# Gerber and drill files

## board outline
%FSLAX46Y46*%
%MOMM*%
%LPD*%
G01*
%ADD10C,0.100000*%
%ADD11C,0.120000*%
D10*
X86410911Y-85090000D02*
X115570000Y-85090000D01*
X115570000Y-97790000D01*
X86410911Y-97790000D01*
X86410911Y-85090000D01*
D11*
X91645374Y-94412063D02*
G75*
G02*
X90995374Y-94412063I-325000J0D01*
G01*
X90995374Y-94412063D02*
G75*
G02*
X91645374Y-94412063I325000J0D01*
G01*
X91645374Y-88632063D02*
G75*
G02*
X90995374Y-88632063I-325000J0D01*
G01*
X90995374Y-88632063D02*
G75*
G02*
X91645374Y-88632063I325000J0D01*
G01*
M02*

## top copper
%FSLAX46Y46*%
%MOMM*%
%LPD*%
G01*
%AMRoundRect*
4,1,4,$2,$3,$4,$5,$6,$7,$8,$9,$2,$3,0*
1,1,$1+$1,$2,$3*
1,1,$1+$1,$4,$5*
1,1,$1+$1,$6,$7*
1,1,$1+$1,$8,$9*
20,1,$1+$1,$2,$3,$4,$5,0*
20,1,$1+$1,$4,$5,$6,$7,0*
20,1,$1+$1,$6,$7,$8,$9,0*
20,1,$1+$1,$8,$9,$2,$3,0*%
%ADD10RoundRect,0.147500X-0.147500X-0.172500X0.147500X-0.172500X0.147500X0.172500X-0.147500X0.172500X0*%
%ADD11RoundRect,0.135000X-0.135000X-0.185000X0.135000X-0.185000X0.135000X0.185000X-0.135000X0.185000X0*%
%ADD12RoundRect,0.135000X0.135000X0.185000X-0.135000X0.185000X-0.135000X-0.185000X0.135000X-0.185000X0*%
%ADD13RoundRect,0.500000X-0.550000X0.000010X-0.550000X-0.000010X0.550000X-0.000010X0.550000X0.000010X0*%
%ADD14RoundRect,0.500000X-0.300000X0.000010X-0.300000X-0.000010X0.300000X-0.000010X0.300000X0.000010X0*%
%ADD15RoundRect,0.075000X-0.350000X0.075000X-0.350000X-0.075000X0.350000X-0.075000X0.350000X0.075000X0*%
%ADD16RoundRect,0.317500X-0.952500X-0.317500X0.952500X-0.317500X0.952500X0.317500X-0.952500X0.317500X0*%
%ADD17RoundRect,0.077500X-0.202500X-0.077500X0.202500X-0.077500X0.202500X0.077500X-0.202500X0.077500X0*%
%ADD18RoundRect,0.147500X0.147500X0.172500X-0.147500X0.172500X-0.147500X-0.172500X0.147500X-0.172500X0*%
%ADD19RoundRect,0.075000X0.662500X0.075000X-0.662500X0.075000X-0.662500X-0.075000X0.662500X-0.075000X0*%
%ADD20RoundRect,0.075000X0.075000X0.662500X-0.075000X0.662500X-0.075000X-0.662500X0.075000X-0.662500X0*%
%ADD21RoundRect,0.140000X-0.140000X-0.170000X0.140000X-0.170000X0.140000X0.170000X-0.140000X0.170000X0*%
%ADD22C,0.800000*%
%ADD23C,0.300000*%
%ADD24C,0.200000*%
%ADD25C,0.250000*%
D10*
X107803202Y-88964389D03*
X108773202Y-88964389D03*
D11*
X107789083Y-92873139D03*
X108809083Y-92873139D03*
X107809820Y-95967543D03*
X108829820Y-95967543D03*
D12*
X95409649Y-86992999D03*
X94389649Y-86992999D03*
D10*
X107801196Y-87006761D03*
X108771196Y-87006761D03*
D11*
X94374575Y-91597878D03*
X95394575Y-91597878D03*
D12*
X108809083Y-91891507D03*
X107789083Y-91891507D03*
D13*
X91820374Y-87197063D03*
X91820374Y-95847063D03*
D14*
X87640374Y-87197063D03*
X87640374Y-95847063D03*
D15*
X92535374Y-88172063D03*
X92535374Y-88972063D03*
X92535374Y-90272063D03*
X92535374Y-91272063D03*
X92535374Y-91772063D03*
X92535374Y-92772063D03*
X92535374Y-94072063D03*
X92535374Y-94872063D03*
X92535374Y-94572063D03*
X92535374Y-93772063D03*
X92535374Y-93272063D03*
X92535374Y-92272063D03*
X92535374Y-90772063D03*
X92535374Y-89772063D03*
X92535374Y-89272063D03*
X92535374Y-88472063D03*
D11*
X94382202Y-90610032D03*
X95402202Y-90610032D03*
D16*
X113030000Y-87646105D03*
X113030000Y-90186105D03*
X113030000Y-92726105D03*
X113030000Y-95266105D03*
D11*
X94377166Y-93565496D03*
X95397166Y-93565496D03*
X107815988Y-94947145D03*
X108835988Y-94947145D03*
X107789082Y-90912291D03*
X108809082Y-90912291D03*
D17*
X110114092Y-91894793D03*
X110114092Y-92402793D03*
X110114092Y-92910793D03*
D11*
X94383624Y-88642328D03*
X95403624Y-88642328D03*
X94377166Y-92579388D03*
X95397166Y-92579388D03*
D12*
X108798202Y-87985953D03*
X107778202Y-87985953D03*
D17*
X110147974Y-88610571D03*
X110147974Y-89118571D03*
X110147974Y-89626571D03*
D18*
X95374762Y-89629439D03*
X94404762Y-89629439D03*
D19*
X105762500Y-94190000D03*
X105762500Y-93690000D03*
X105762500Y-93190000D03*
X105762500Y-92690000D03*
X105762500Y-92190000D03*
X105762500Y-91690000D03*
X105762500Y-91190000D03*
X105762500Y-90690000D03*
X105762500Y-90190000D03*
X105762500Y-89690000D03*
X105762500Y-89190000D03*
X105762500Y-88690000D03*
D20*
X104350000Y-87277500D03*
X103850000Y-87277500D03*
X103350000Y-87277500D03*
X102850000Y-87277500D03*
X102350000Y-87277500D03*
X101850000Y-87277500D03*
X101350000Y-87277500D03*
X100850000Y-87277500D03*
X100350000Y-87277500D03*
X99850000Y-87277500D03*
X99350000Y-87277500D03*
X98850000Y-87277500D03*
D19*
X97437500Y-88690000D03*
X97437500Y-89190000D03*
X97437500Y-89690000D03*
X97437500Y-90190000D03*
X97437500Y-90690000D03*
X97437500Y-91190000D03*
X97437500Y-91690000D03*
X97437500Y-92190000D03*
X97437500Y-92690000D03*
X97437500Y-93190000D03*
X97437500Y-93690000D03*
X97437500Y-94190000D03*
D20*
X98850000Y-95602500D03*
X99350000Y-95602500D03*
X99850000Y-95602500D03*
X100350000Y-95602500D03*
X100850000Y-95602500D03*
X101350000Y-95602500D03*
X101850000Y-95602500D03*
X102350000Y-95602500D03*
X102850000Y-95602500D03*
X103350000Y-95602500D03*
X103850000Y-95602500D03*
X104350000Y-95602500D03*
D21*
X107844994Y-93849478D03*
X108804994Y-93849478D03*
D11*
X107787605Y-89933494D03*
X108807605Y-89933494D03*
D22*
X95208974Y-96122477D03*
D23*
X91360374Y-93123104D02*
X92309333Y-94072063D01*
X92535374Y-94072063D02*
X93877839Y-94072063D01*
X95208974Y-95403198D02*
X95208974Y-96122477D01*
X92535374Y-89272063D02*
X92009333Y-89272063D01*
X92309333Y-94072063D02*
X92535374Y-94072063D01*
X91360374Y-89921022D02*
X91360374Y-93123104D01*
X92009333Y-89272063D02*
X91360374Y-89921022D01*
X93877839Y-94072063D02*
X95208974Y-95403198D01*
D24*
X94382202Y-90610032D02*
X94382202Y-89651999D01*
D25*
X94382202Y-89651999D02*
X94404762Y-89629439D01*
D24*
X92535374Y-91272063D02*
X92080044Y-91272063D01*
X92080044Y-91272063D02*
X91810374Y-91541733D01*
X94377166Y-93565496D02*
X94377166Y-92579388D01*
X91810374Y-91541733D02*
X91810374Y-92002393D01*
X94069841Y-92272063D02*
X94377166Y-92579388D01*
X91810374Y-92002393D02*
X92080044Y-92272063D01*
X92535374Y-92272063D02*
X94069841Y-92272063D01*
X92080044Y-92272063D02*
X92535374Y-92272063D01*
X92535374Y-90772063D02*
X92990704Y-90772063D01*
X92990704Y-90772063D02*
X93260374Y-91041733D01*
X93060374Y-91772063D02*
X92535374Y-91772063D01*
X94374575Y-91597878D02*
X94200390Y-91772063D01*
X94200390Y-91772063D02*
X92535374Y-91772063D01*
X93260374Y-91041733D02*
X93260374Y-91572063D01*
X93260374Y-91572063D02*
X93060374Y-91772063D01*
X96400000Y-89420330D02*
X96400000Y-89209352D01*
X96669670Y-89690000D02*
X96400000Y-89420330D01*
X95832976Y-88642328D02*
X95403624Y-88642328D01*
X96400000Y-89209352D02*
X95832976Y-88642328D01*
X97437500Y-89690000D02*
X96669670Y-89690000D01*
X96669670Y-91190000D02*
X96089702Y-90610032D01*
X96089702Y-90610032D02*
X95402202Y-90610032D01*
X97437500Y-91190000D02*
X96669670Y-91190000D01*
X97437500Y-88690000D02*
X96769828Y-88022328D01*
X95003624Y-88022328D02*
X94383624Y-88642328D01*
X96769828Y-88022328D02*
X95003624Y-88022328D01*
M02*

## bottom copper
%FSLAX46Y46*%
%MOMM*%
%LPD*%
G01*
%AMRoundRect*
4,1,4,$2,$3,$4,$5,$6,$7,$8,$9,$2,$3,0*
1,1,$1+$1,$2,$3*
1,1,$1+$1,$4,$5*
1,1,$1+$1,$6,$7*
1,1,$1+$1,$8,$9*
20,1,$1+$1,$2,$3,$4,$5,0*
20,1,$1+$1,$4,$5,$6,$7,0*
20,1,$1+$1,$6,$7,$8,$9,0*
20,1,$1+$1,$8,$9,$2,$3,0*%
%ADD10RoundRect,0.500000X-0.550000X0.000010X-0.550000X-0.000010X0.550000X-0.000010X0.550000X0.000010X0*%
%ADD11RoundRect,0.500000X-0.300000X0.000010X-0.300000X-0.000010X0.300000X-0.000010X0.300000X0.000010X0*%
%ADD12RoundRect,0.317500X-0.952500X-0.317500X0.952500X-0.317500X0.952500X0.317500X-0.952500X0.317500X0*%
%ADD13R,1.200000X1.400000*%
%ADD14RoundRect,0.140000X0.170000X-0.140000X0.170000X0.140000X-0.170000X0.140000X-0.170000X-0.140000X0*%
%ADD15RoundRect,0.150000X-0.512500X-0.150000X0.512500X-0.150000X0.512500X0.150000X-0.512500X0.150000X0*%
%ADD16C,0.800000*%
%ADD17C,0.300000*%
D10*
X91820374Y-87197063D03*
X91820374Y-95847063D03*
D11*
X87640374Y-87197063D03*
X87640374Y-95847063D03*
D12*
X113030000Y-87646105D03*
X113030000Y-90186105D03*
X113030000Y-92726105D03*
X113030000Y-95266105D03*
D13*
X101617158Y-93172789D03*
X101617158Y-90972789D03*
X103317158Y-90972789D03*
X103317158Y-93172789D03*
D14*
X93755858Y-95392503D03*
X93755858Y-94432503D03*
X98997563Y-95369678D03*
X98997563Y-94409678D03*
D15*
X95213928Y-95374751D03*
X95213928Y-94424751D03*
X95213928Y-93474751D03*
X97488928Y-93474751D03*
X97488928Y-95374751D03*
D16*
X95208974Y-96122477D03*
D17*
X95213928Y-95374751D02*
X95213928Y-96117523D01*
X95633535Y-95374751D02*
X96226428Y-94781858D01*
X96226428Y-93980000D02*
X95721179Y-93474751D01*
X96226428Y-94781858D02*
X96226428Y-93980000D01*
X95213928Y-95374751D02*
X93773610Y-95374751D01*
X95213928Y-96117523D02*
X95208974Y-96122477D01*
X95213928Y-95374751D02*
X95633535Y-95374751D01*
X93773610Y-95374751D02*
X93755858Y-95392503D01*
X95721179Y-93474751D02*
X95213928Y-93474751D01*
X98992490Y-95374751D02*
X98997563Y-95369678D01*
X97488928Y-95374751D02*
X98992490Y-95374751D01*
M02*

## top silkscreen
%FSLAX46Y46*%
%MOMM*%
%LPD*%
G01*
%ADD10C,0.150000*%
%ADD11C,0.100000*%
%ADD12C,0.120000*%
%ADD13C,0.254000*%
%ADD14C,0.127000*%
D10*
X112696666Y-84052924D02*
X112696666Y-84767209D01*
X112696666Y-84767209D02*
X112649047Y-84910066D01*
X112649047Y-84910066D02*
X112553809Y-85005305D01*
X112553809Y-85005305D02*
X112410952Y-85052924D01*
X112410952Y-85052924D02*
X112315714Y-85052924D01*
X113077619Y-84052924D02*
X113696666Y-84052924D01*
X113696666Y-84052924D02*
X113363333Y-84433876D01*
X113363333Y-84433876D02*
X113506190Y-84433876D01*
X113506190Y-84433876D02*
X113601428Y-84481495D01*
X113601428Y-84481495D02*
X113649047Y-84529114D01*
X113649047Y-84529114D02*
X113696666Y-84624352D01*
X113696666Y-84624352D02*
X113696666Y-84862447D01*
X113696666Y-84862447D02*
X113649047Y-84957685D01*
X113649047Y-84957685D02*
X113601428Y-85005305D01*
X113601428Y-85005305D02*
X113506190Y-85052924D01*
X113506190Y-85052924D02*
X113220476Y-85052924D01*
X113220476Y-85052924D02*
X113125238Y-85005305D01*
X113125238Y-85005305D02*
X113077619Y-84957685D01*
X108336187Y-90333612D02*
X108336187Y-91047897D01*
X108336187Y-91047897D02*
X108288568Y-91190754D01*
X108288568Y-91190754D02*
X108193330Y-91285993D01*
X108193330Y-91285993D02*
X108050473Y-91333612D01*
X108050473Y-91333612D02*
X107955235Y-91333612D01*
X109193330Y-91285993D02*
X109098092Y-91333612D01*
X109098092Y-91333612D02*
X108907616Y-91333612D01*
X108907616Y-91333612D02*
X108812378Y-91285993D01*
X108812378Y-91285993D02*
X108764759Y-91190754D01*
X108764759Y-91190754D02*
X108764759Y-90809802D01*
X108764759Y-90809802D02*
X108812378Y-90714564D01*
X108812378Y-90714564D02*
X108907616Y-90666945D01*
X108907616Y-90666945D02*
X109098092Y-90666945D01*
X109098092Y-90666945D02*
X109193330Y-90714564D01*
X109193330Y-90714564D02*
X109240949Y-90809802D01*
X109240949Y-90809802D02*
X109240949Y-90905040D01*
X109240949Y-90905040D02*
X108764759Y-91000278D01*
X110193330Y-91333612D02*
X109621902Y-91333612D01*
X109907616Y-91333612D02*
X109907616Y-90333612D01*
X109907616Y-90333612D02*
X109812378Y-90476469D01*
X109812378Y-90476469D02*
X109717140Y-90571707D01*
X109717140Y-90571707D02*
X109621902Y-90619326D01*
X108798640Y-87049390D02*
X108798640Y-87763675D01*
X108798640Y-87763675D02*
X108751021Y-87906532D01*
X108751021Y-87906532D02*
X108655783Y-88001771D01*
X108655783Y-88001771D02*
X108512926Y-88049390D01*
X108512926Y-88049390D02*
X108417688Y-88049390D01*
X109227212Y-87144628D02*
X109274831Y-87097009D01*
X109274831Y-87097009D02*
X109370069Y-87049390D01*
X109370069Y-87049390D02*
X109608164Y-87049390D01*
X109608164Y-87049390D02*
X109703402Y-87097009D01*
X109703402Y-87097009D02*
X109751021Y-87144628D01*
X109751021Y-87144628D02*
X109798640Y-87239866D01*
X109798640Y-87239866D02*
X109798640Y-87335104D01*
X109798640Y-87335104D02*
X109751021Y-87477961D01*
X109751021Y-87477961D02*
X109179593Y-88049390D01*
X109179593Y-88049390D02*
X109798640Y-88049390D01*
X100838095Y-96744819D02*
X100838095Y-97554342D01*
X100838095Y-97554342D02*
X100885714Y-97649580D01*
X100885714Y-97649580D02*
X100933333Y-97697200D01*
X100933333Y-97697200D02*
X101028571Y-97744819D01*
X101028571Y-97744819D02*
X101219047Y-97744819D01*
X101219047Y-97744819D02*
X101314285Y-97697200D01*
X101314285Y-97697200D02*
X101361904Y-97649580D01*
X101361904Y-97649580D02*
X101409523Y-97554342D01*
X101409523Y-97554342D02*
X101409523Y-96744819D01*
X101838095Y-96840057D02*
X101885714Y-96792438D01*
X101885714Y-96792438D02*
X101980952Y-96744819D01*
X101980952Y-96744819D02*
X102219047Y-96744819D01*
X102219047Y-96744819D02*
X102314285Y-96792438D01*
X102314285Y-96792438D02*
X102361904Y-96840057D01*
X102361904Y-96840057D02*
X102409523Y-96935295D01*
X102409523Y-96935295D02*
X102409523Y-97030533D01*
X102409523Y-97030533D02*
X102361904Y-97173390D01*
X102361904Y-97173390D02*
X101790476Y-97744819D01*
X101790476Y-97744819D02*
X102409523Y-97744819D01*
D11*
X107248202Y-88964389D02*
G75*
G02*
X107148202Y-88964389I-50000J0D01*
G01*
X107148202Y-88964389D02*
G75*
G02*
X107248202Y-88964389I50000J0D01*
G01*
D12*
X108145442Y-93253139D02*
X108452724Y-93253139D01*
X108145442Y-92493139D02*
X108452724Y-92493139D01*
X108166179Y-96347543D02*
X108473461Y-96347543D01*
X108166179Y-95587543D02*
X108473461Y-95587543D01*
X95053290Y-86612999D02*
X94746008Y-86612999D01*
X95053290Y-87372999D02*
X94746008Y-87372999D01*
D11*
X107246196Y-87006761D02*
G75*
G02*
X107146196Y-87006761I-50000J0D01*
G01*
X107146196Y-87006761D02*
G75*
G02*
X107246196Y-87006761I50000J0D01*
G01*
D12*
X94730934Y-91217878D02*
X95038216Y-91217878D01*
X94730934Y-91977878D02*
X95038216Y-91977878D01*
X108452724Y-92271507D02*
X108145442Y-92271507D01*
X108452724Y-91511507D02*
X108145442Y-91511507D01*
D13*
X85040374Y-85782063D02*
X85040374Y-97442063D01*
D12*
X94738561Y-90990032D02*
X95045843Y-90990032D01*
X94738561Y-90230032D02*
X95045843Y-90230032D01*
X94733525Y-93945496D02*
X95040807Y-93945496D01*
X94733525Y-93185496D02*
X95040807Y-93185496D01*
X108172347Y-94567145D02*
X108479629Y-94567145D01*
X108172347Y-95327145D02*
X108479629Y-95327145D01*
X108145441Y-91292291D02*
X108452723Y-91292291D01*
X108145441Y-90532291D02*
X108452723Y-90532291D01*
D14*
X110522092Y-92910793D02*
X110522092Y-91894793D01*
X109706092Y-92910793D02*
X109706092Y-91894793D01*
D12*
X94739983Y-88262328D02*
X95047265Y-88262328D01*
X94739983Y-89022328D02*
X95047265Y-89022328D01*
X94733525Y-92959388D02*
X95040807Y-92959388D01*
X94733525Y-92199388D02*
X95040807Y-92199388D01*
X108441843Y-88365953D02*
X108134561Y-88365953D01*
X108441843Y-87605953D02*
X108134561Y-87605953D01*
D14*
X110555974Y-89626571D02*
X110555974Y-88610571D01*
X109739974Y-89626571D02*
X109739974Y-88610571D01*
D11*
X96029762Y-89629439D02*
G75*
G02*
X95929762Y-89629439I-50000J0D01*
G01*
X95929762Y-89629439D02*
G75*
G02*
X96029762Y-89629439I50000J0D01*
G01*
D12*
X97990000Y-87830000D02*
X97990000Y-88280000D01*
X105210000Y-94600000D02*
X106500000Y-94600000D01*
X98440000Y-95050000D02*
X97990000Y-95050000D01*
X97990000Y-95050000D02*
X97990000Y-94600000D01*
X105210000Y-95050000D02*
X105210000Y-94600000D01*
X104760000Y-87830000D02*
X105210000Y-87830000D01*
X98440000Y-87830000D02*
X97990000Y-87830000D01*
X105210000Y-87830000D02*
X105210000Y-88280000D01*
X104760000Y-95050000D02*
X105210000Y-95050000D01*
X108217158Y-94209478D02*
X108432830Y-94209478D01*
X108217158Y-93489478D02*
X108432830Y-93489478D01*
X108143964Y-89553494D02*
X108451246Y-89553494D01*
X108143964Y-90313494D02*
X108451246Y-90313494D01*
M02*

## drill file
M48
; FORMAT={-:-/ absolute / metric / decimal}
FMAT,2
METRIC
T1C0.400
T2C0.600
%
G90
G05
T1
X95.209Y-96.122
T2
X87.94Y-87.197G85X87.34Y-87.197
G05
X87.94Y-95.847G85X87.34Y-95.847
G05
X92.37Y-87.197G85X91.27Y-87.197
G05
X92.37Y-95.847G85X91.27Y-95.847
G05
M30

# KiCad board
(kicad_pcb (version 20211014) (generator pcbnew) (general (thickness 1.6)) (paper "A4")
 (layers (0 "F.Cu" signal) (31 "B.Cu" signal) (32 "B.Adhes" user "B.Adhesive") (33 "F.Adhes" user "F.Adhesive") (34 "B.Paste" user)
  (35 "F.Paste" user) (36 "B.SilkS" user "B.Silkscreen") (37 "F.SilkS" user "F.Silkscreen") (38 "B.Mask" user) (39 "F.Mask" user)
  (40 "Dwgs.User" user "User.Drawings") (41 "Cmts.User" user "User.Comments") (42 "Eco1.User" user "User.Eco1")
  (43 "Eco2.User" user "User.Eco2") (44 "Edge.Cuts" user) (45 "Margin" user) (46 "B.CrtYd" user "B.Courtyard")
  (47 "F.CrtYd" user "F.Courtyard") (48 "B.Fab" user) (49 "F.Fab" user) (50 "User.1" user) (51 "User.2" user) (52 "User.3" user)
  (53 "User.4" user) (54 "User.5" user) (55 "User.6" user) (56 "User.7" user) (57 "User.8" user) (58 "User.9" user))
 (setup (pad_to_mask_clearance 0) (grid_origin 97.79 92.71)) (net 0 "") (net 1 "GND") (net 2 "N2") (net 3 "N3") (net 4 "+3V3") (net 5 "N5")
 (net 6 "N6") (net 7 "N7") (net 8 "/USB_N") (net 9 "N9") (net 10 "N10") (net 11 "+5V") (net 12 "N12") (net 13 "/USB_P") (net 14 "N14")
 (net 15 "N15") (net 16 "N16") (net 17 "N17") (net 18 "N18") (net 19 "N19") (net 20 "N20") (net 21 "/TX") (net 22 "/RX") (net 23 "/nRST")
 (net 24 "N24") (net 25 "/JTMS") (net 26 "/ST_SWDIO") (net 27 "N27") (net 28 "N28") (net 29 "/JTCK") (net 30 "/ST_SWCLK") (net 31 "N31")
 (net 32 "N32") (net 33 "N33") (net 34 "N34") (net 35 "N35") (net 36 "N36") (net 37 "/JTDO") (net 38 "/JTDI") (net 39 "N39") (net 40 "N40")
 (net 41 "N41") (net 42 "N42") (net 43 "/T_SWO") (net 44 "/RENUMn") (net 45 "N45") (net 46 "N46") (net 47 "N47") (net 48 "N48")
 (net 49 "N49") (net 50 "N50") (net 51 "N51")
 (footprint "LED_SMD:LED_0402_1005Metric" (layer "F.Cu") (at 108.288202 88.964389)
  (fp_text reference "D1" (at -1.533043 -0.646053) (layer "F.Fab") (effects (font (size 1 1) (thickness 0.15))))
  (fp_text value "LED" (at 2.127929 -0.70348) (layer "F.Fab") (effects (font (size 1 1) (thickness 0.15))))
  (fp_circle (center -1.09 0) (end -1.04 0) (layer "F.SilkS") (width 0.1) (fill none))
  (pad "1" smd roundrect (at -0.485 0) (size 0.59 0.64) (layers "F.Cu" "F.Paste" "F.Mask") (roundrect_rratio 0.25) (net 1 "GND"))
  (pad "2" smd roundrect (at 0.485 0) (size 0.59 0.64) (layers "F.Cu" "F.Paste" "F.Mask") (roundrect_rratio 0.25) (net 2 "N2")))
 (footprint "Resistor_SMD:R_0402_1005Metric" (layer "F.Cu") (at 108.299083 92.873139)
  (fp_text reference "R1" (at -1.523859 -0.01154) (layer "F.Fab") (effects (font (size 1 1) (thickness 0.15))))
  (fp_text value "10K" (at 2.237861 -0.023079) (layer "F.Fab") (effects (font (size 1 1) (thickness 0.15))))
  (fp_line (start -0.153641 0.38) (end 0.153641 0.38) (layer "F.SilkS") (width 0.12))
  (fp_line (start -0.153641 -0.38) (end 0.153641 -0.38) (layer "F.SilkS") (width 0.12))
  (pad "1" smd roundrect (at -0.51 0) (size 0.54 0.64) (layers "F.Cu" "F.Paste" "F.Mask") (roundrect_rratio 0.25) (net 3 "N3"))
  (pad "2" smd roundrect (at 0.51 0) (size 0.54 0.64) (layers "F.Cu" "F.Paste" "F.Mask") (roundrect_rratio 0.25) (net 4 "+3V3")))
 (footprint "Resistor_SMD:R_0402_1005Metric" (layer "F.Cu") (at 108.31982 95.967543)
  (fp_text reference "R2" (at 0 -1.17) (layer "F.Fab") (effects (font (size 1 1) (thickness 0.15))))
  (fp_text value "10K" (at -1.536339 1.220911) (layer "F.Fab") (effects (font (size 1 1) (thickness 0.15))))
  (fp_line (start -0.153641 0.38) (end 0.153641 0.38) (layer "F.SilkS") (width 0.12))
  (fp_line (start -0.153641 -0.38) (end 0.153641 -0.38) (layer "F.SilkS") (width 0.12))
  (pad "1" smd roundrect (at -0.51 0) (size 0.54 0.64) (layers "F.Cu" "F.Paste" "F.Mask") (roundrect_rratio 0.25) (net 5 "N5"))
  (pad "2" smd roundrect (at 0.51 0) (size 0.54 0.64) (layers "F.Cu" "F.Paste" "F.Mask") (roundrect_rratio 0.25) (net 1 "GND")))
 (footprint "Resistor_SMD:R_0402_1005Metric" (layer "F.Cu") (at 94.899649 86.992999 180)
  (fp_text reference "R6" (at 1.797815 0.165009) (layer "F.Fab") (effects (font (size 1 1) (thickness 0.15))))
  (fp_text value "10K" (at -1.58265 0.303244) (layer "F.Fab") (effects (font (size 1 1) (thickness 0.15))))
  (fp_line (start -0.153641 0.38) (end 0.153641 0.38) (layer "F.SilkS") (width 0.12))
  (fp_line (start -0.153641 -0.38) (end 0.153641 -0.38) (layer "F.SilkS") (width 0.12))
  (pad "1" smd roundrect (at -0.51 0 180) (size 0.54 0.64) (layers "F.Cu" "F.Paste" "F.Mask") (roundrect_rratio 0.25) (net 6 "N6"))
  (pad "2" smd roundrect (at 0.51 0 180) (size 0.54 0.64) (layers "F.Cu" "F.Paste" "F.Mask") (roundrect_rratio 0.25) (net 1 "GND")))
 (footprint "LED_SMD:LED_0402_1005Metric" (layer "F.Cu") (at 108.286196 87.006761)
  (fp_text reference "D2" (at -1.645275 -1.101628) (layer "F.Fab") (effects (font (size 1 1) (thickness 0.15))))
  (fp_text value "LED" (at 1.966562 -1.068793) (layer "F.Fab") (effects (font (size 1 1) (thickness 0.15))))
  (fp_circle (center -1.09 0) (end -1.04 0) (layer "F.SilkS") (width 0.1) (fill none))
  (pad "1" smd roundrect (at -0.485 0) (size 0.59 0.64) (layers "F.Cu" "F.Paste" "F.Mask") (roundrect_rratio 0.25) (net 1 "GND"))
  (pad "2" smd roundrect (at 0.485 0) (size 0.59 0.64) (layers "F.Cu" "F.Paste" "F.Mask") (roundrect_rratio 0.25) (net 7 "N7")))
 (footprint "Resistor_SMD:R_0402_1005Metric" (layer "F.Cu") (at 94.884575 91.597878)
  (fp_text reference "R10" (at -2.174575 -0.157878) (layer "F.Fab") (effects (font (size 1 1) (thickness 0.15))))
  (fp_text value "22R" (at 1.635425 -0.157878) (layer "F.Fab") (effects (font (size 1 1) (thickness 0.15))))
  (fp_line (start -0.153641 -0.38) (end 0.153641 -0.38) (layer "F.SilkS") (width 0.12))
  (fp_line (start -0.153641 0.38) (end 0.153641 0.38) (layer "F.SilkS") (width 0.12))
  (pad "1" smd roundrect (at -0.51 0) (size 0.54 0.64) (layers "F.Cu" "F.Paste" "F.Mask") (roundrect_rratio 0.25) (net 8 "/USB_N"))
  (pad "2" smd roundrect (at 0.51 0) (size 0.54 0.64) (layers "F.Cu" "F.Paste" "F.Mask") (roundrect_rratio 0.25) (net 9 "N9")))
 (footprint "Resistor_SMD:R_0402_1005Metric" (layer "F.Cu") (at 108.299083 91.891507 180)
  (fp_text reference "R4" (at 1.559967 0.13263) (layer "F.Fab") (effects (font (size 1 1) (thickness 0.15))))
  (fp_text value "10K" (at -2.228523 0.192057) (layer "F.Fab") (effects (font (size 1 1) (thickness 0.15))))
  (fp_line (start -0.153641 -0.38) (end 0.153641 -0.38) (layer "F.SilkS") (width 0.12))
  (fp_line (start -0.153641 0.38) (end 0.153641 0.38) (layer "F.SilkS") (width 0.12))
  (pad "1" smd roundrect (at -0.51 0 180) (size 0.54 0.64) (layers "F.Cu" "F.Paste" "F.Mask") (roundrect_rratio 0.25) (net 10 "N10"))
  (pad "2" smd roundrect (at 0.51 0 180) (size 0.54 0.64) (layers "F.Cu" "F.Paste" "F.Mask") (roundrect_rratio 0.25) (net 4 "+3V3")))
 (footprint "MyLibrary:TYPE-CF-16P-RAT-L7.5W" (layer "F.Cu") (at 92.535374 88.322063 -90)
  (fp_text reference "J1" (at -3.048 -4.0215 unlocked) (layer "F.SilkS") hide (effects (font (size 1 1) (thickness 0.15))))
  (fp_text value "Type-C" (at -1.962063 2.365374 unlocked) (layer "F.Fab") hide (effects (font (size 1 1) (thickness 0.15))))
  (fp_line (start -2.54 7.495) (end 9.12 7.495) (layer "F.SilkS") (width 0.254))
  (fp_circle (center 6.09 1.215) (end 6.415 1.215) (layer "Edge.Cuts") (width 0.12) (fill none))
  (fp_circle (center 0.31 1.215) (end 0.635 1.215) (layer "Edge.Cuts") (width 0.12) (fill none))
  (pad "1" thru_hole roundrect (at -1.125 0.715 270) (size 1 2.1) (drill oval 0.6 1.7) (layers *.Cu *.Mask) (roundrect_rratio 0.5)
   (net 1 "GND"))
  (pad "2" thru_hole roundrect (at 7.525 0.715 270) (size 1 2.1) (drill oval 0.6 1.7) (layers *.Cu *.Mask) (roundrect_rratio 0.5)
   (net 1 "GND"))
  (pad "3" thru_hole roundrect (at -1.125 4.895 270) (size 1 1.6) (drill oval 0.6 1.2) (layers *.Cu *.Mask) (roundrect_rratio 0.5)
   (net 1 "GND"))
  (pad "4" thru_hole roundrect (at 7.525 4.895 270) (size 1 1.6) (drill oval 0.6 1.2) (layers *.Cu *.Mask) (roundrect_rratio 0.5)
   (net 1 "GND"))
  (pad "A1" smd roundrect (at -0.15 0 270) (size 0.3 0.85) (layers "F.Cu" "F.Paste" "F.Mask") (roundrect_rratio 0.25) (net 1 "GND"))
  (pad "A4" smd roundrect (at 0.65 0 270) (size 0.3 0.85) (layers "F.Cu" "F.Paste" "F.Mask") (roundrect_rratio 0.25) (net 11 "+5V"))
  (pad "A5" smd roundrect (at 1.95 0 270) (size 0.3 0.85) (layers "F.Cu" "F.Paste" "F.Mask") (roundrect_rratio 0.25) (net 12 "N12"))
  (pad "A6" smd roundrect (at 2.95 0 270) (size 0.3 0.85) (layers "F.Cu" "F.Paste" "F.Mask") (roundrect_rratio 0.25) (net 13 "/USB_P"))
  (pad "A7" smd roundrect (at 3.45 0 270) (size 0.3 0.85) (layers "F.Cu" "F.Paste" "F.Mask") (roundrect_rratio 0.25) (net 8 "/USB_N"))
  (pad "A8" smd roundrect (at 4.45 0 270) (size 0.3 0.85) (layers "F.Cu" "F.Paste" "F.Mask") (roundrect_rratio 0.25) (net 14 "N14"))
  (pad "A9" smd roundrect (at 5.75 0 270) (size 0.3 0.85) (layers "F.Cu" "F.Paste" "F.Mask") (roundrect_rratio 0.25) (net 11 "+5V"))
  (pad "A12" smd roundrect (at 6.55 0 270) (size 0.3 0.85) (layers "F.Cu" "F.Paste" "F.Mask") (roundrect_rratio 0.25) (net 1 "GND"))
  (pad "B1" smd roundrect (at 6.25 0 270) (size 0.3 0.85) (layers "F.Cu" "F.Paste" "F.Mask") (roundrect_rratio 0.25) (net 1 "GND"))
  (pad "B4" smd roundrect (at 5.45 0 270) (size 0.3 0.85) (layers "F.Cu" "F.Paste" "F.Mask") (roundrect_rratio 0.25) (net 11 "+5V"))
  (pad "B5" smd roundrect (at 4.95 0 270) (size 0.3 0.85) (layers "F.Cu" "F.Paste" "F.Mask") (roundrect_rratio 0.25) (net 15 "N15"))
  (pad "B6" smd roundrect (at 3.95 0 270) (size 0.3 0.85) (layers "F.Cu" "F.Paste" "F.Mask") (roundrect_rratio 0.25) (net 13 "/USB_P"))
  (pad "B7" smd roundrect (at 2.45 0 270) (size 0.3 0.85) (layers "F.Cu" "F.Paste" "F.Mask") (roundrect_rratio 0.25) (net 8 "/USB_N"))
  (pad "B8" smd roundrect (at 1.45 0 270) (size 0.3 0.85) (layers "F.Cu" "F.Paste" "F.Mask") (roundrect_rratio 0.25) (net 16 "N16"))
  (pad "B9" smd roundrect (at 0.95 0 270) (size 0.3 0.85) (layers "F.Cu" "F.Paste" "F.Mask") (roundrect_rratio 0.25) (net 11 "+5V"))
  (pad "B12" smd roundrect (at 0.15 0 270) (size 0.3 0.85) (layers "F.Cu" "F.Paste" "F.Mask") (roundrect_rratio 0.25) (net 1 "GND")))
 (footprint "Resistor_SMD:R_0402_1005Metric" (layer "F.Cu") (at 94.892202 90.610032)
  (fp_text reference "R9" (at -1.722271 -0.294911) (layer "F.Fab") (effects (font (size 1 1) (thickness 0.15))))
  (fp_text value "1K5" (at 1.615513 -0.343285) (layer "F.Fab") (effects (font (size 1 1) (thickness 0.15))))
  (fp_line (start -0.153641 0.38) (end 0.153641 0.38) (layer "F.SilkS") (width 0.12))
  (fp_line (start -0.153641 -0.38) (end 0.153641 -0.38) (layer "F.SilkS") (width 0.12))
  (pad "1" smd roundrect (at -0.51 0) (size 0.54 0.64) (layers "F.Cu" "F.Paste" "F.Mask") (roundrect_rratio 0.25) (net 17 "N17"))
  (pad "2" smd roundrect (at 0.51 0) (size 0.54 0.64) (layers "F.Cu" "F.Paste" "F.Mask") (roundrect_rratio 0.25) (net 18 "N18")))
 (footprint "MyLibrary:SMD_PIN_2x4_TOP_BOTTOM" (layer "F.Cu") (at 113.03 87.646105)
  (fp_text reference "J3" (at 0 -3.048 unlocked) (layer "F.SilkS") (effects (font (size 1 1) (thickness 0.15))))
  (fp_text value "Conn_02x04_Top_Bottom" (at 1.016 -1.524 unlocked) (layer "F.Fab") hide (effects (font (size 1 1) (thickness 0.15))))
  (pad "1" smd roundrect (at 0 0) (size 2.54 1.27) (layers "F.Cu" "F.Paste" "F.Mask") (roundrect_rratio 0.25) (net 4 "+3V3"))
  (pad "2" smd roundrect (at 0 2.54) (size 2.54 1.27) (layers "F.Cu" "F.Paste" "F.Mask") (roundrect_rratio 0.25) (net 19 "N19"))
  (pad "3" smd roundrect (at 0 5.08) (size 2.54 1.27) (layers "F.Cu" "F.Paste" "F.Mask") (roundrect_rratio 0.25) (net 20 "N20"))
  (pad "4" smd roundrect (at 0 7.62) (size 2.54 1.27) (layers "F.Cu" "F.Paste" "F.Mask") (roundrect_rratio 0.25) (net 1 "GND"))
  (pad "5" smd roundrect (at 0 0) (size 2.54 1.27) (layers "B.Cu" "B.Paste" "B.Mask") (roundrect_rratio 0.25) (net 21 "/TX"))
  (pad "6" smd roundrect (at 0 2.54) (size 2.54 1.27) (layers "B.Cu" "B.Paste" "B.Mask") (roundrect_rratio 0.25) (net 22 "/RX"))
  (pad "7" smd roundrect (at 0 5.08) (size 2.54 1.27) (layers "B.Cu" "B.Paste" "B.Mask") (roundrect_rratio 0.25) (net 11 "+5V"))
  (pad "8" smd roundrect (at 0 7.62) (size 2.54 1.27) (layers "B.Cu" "B.Paste" "B.Mask") (roundrect_rratio 0.25) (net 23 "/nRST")))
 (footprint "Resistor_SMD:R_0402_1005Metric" (layer "F.Cu") (at 94.887166 93.565496)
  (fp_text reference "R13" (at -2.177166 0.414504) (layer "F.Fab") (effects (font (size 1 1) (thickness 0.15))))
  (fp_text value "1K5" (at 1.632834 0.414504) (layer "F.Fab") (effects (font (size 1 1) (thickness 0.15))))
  (fp_line (start -0.153641 0.38) (end 0.153641 0.38) (layer "F.SilkS") (width 0.12))
  (fp_line (start -0.153641 -0.38) (end 0.153641 -0.38) (layer "F.SilkS") (width 0.12))
  (pad "1" smd roundrect (at -0.51 0) (size 0.54 0.64) (layers "F.Cu" "F.Paste" "F.Mask") (roundrect_rratio 0.25) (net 13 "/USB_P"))
  (pad "2" smd roundrect (at 0.51 0) (size 0.54 0.64) (layers "F.Cu" "F.Paste" "F.Mask") (roundrect_rratio 0.25) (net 4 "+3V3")))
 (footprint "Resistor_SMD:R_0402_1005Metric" (layer "F.Cu") (at 108.325988 94.947145)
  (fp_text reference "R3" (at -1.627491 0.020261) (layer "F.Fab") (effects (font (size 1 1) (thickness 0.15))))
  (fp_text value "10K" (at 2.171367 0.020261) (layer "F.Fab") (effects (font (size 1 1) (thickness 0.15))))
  (fp_line (start -0.153641 -0.38) (end 0.153641 -0.38) (layer "F.SilkS") (width 0.12))
  (fp_line (start -0.153641 0.38) (end 0.153641 0.38) (layer "F.SilkS") (width 0.12))
  (pad "1" smd roundrect (at -0.51 0) (size 0.54 0.64) (layers "F.Cu" "F.Paste" "F.Mask") (roundrect_rratio 0.25) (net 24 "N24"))
  (pad "2" smd roundrect (at 0.51 0) (size 0.54 0.64) (layers "F.Cu" "F.Paste" "F.Mask") (roundrect_rratio 0.25) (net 1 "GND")))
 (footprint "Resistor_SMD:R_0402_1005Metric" (layer "F.Cu") (at 108.299082 90.912291)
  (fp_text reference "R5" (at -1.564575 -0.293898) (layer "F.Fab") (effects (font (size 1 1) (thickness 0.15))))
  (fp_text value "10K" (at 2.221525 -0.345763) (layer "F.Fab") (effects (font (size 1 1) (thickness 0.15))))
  (fp_line (start -0.153641 0.38) (end 0.153641 0.38) (layer "F.SilkS") (width 0.12))
  (fp_line (start -0.153641 -0.38) (end 0.153641 -0.38) (layer "F.SilkS") (width 0.12))
  (pad "1" smd roundrect (at -0.51 0) (size 0.54 0.64) (layers "F.Cu" "F.Paste" "F.Mask") (roundrect_rratio 0.25) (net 1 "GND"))
  (pad "2" smd roundrect (at 0.51 0) (size 0.54 0.64) (layers "F.Cu" "F.Paste" "F.Mask") (roundrect_rratio 0.25) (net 10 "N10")))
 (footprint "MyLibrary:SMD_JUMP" (layer "F.Cu") (at 110.114092 92.402793)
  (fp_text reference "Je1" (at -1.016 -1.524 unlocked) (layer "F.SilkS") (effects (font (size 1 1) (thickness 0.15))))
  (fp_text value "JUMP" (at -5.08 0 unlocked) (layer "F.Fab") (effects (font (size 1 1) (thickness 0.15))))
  (fp_line (start 0.408 0.508) (end 0.408 -0.508) (layer "F.SilkS") (width 0.127))
  (fp_line (start -0.408 0.508) (end -0.408 -0.508) (layer "F.SilkS") (width 0.127))
  (pad "1" smd roundrect (at 0 -0.508) (size 0.56 0.31) (layers "F.Cu" "F.Paste" "F.Mask") (roundrect_rratio 0.25) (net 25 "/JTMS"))
  (pad "2" smd roundrect (at 0 0) (size 0.56 0.31) (layers "F.Cu" "F.Paste" "F.Mask") (roundrect_rratio 0.25) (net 20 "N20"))
  (pad "3" smd roundrect (at 0 0.508) (size 0.56 0.31) (layers "F.Cu" "F.Paste" "F.Mask") (roundrect_rratio 0.25) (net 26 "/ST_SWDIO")))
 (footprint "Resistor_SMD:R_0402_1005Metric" (layer "F.Cu") (at 94.893624 88.642328)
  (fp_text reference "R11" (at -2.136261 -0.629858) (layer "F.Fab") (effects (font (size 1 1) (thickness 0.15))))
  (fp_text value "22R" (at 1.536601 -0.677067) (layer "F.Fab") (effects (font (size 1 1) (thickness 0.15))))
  (fp_line (start -0.153641 -0.38) (end 0.153641 -0.38) (layer "F.SilkS") (width 0.12))
  (fp_line (start -0.153641 0.38) (end 0.153641 0.38) (layer "F.SilkS") (width 0.12))
  (pad "1" smd roundrect (at -0.51 0) (size 0.54 0.64) (layers "F.Cu" "F.Paste" "F.Mask") (roundrect_rratio 0.25) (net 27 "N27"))
  (pad "2" smd roundrect (at 0.51 0) (size 0.54 0.64) (layers "F.Cu" "F.Paste" "F.Mask") (roundrect_rratio 0.25) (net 25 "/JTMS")))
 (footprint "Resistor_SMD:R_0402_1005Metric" (layer "F.Cu") (at 94.887166 92.579388)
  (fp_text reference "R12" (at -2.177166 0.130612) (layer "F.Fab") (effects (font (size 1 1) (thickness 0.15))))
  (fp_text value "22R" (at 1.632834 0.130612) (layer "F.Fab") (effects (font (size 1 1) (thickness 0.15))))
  (fp_line (start -0.153641 0.38) (end 0.153641 0.38) (layer "F.SilkS") (width 0.12))
  (fp_line (start -0.153641 -0.38) (end 0.153641 -0.38) (layer "F.SilkS") (width 0.12))
  (pad "1" smd roundrect (at -0.51 0) (size 0.54 0.64) (layers "F.Cu" "F.Paste" "F.Mask") (roundrect_rratio 0.25) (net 13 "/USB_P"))
  (pad "2" smd roundrect (at 0.51 0) (size 0.54 0.64) (layers "F.Cu" "F.Paste" "F.Mask") (roundrect_rratio 0.25) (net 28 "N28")))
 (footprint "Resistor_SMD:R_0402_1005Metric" (layer "F.Cu") (at 108.288202 87.985953 180)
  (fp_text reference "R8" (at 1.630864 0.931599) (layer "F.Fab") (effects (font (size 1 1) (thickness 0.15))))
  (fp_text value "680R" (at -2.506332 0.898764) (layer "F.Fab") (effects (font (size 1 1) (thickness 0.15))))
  (fp_line (start -0.153641 -0.38) (end 0.153641 -0.38) (layer "F.SilkS") (width 0.12))
  (fp_line (start -0.153641 0.38) (end 0.153641 0.38) (layer "F.SilkS") (width 0.12))
  (pad "1" smd roundrect (at -0.51 0 180) (size 0.54 0.64) (layers "F.Cu" "F.Paste" "F.Mask") (roundrect_rratio 0.25) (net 7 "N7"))
  (pad "2" smd roundrect (at 0.51 0 180) (size 0.54 0.64) (layers "F.Cu" "F.Paste" "F.Mask") (roundrect_rratio 0.25) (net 22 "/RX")))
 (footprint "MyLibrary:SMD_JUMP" (layer "F.Cu") (at 110.147974 89.118571)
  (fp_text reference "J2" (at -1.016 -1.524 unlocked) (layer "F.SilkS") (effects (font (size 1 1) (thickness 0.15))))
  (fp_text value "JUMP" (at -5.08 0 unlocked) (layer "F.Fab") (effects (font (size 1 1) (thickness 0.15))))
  (fp_line (start 0.408 0.508) (end 0.408 -0.508) (layer "F.SilkS") (width 0.127))
  (fp_line (start -0.408 0.508) (end -0.408 -0.508) (layer "F.SilkS") (width 0.127))
  (pad "1" smd roundrect (at 0 -0.508) (size 0.56 0.31) (layers "F.Cu" "F.Paste" "F.Mask") (roundrect_rratio 0.25) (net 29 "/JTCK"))
  (pad "2" smd roundrect (at 0 0) (size 0.56 0.31) (layers "F.Cu" "F.Paste" "F.Mask") (roundrect_rratio 0.25) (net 19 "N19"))
  (pad "3" smd roundrect (at 0 0.508) (size 0.56 0.31) (layers "F.Cu" "F.Paste" "F.Mask") (roundrect_rratio 0.25) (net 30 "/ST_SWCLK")))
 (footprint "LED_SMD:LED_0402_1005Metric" (layer "F.Cu") (at 94.889762 89.629439 180)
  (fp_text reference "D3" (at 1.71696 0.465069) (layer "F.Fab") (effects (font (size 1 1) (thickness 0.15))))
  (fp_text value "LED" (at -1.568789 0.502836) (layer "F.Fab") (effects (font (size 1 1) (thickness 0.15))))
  (fp_circle (center -1.09 0) (end -1.04 0) (layer "F.SilkS") (width 0.1) (fill none))
  (pad "1" smd roundrect (at -0.485 0 180) (size 0.59 0.64) (layers "F.Cu" "F.Paste" "F.Mask") (roundrect_rratio 0.25) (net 1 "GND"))
  (pad "2" smd roundrect (at 0.485 0 180) (size 0.59 0.64) (layers "F.Cu" "F.Paste" "F.Mask") (roundrect_rratio 0.25) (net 17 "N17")))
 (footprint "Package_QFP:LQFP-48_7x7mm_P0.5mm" (layer "F.Cu") (at 101.6 91.44 180)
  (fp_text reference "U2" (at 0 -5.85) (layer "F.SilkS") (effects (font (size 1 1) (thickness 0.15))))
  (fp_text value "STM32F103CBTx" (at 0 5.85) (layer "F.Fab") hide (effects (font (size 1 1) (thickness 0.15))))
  (fp_line (start 3.61 3.61) (end 3.61 3.16) (layer "F.SilkS") (width 0.12))
  (fp_line (start -3.61 -3.16) (end -4.9 -3.16) (layer "F.SilkS") (width 0.12))
  (fp_line (start 3.16 -3.61) (end 3.61 -3.61) (layer "F.SilkS") (width 0.12))
  (fp_line (start 3.61 -3.61) (end 3.61 -3.16) (layer "F.SilkS") (width 0.12))
  (fp_line (start -3.61 -3.61) (end -3.61 -3.16) (layer "F.SilkS") (width 0.12))
  (fp_line (start -3.16 3.61) (end -3.61 3.61) (layer "F.SilkS") (width 0.12))
  (fp_line (start 3.16 3.61) (end 3.61 3.61) (layer "F.SilkS") (width 0.12))
  (fp_line (start -3.61 3.61) (end -3.61 3.16) (layer "F.SilkS") (width 0.12))
  (fp_line (start -3.16 -3.61) (end -3.61 -3.61) (layer "F.SilkS") (width 0.12))
  (pad "1" smd roundrect (at -4.1625 -2.75 180) (size 1.475 0.3) (layers "F.Cu" "F.Paste" "F.Mask") (roundrect_rratio 0.25) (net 4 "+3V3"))
  (pad "2" smd roundrect (at -4.1625 -2.25 180) (size 1.475 0.3) (layers "F.Cu" "F.Paste" "F.Mask") (roundrect_rratio 0.25) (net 24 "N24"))
  (pad "3" smd roundrect (at -4.1625 -1.75 180) (size 1.475 0.3) (layers "F.Cu" "F.Paste" "F.Mask") (roundrect_rratio 0.25) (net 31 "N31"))
  (pad "4" smd roundrect (at -4.1625 -1.25 180) (size 1.475 0.3) (layers "F.Cu" "F.Paste" "F.Mask") (roundrect_rratio 0.25) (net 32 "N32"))
  (pad "5" smd roundrect (at -4.1625 -0.75 180) (size 1.475 0.3) (layers "F.Cu" "F.Paste" "F.Mask") (roundrect_rratio 0.25) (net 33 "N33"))
  (pad "6" smd roundrect (at -4.1625 -0.25 180) (size 1.475 0.3) (layers "F.Cu" "F.Paste" "F.Mask") (roundrect_rratio 0.25) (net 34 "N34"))
  (pad "7" smd roundrect (at -4.1625 0.25 180) (size 1.475 0.3) (layers "F.Cu" "F.Paste" "F.Mask") (roundrect_rratio 0.25) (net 3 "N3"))
  (pad "8" smd roundrect (at -4.1625 0.75 180) (size 1.475 0.3) (layers "F.Cu" "F.Paste" "F.Mask") (roundrect_rratio 0.25) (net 1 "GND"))
  (pad "9" smd roundrect (at -4.1625 1.25 180) (size 1.475 0.3) (layers "F.Cu" "F.Paste" "F.Mask") (roundrect_rratio 0.25) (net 4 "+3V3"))
  (pad "10" smd roundrect (at -4.1625 1.75 180) (size 1.475 0.3) (layers "F.Cu" "F.Paste" "F.Mask") (roundrect_rratio 0.25) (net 10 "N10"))
  (pad "11" smd roundrect (at -4.1625 2.25 180) (size 1.475 0.3) (layers "F.Cu" "F.Paste" "F.Mask") (roundrect_rratio 0.25) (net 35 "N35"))
  (pad "12" smd roundrect (at -4.1625 2.75 180) (size 1.475 0.3) (layers "F.Cu" "F.Paste" "F.Mask") (roundrect_rratio 0.25) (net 21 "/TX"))
  (pad "13" smd roundrect (at -2.75 4.1625 180) (size 0.3 1.475) (layers "F.Cu" "F.Paste" "F.Mask") (roundrect_rratio 0.25) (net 22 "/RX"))
  (pad "14" smd roundrect (at -2.25 4.1625 180) (size 0.3 1.475) (layers "F.Cu" "F.Paste" "F.Mask") (roundrect_rratio 0.25) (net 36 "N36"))
  (pad "15" smd roundrect (at -1.75 4.1625 180) (size 0.3 1.475) (layers "F.Cu" "F.Paste" "F.Mask") (roundrect_rratio 0.25) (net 29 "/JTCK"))
  (pad "16" smd roundrect (at -1.25 4.1625 180) (size 0.3 1.475) (layers "F.Cu" "F.Paste" "F.Mask") (roundrect_rratio 0.25) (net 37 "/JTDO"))
  (pad "17" smd roundrect (at -0.75 4.1625 180) (size 0.3 1.475) (layers "F.Cu" "F.Paste" "F.Mask") (roundrect_rratio 0.25) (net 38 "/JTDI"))
  (pad "18" smd roundrect (at -0.25 4.1625 180) (size 0.3 1.475) (layers "F.Cu" "F.Paste" "F.Mask") (roundrect_rratio 0.25) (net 23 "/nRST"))
  (pad "19" smd roundrect (at 0.25 4.1625 180) (size 0.3 1.475) (layers "F.Cu" "F.Paste" "F.Mask") (roundrect_rratio 0.25) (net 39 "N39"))
  (pad "20" smd roundrect (at 0.75 4.1625 180) (size 0.3 1.475) (layers "F.Cu" "F.Paste" "F.Mask") (roundrect_rratio 0.25) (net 6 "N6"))
  (pad "21" smd roundrect (at 1.25 4.1625 180) (size 0.3 1.475) (layers "F.Cu" "F.Paste" "F.Mask") (roundrect_rratio 0.25) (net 1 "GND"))
  (pad "22" smd roundrect (at 1.75 4.1625 180) (size 0.3 1.475) (layers "F.Cu" "F.Paste" "F.Mask") (roundrect_rratio 0.25) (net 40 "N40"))
  (pad "23" smd roundrect (at 2.25 4.1625 180) (size 0.3 1.475) (layers "F.Cu" "F.Paste" "F.Mask") (roundrect_rratio 0.25) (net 1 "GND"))
  (pad "24" smd roundrect (at 2.75 4.1625 180) (size 0.3 1.475) (layers "F.Cu" "F.Paste" "F.Mask") (roundrect_rratio 0.25) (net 4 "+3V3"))
  (pad "25" smd roundrect (at 4.1625 2.75 180) (size 1.475 0.3) (layers "F.Cu" "F.Paste" "F.Mask") (roundrect_rratio 0.25) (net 27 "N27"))
  (pad "26" smd roundrect (at 4.1625 2.25 180) (size 1.475 0.3) (layers "F.Cu" "F.Paste" "F.Mask") (roundrect_rratio 0.25) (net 29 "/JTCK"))
  (pad "27" smd roundrect (at 4.1625 1.75 180) (size 1.475 0.3) (layers "F.Cu" "F.Paste" "F.Mask") (roundrect_rratio 0.25) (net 25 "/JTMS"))
  (pad "28" smd roundrect (at 4.1625 1.25 180) (size 1.475 0.3) (layers "F.Cu" "F.Paste" "F.Mask") (roundrect_rratio 0.25) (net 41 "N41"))
  (pad "29" smd roundrect (at 4.1625 0.75 180) (size 1.475 0.3) (layers "F.Cu" "F.Paste" "F.Mask") (roundrect_rratio 0.25) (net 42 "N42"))
  (pad "30" smd roundrect (at 4.1625 0.25 180) (size 1.475 0.3) (layers "F.Cu" "F.Paste" "F.Mask") (roundrect_rratio 0.25) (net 18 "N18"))
  (pad "31" smd roundrect (at 4.1625 -0.25 180) (size 1.475 0.3) (layers "F.Cu" "F.Paste" "F.Mask") (roundrect_rratio 0.25)
   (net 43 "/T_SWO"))
  (pad "32" smd roundrect (at 4.1625 -0.75 180) (size 1.475 0.3) (layers "F.Cu" "F.Paste" "F.Mask") (roundrect_rratio 0.25) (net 9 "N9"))
  (pad "33" smd roundrect (at 4.1625 -1.25 180) (size 1.475 0.3) (layers "F.Cu" "F.Paste" "F.Mask") (roundrect_rratio 0.25) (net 28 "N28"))
  (pad "34" smd roundrect (at 4.1625 -1.75 180) (size 1.475 0.3) (layers "F.Cu" "F.Paste" "F.Mask") (roundrect_rratio 0.25)
   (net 26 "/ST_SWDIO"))
  (pad "35" smd roundrect (at 4.1625 -2.25 180) (size 1.475 0.3) (layers "F.Cu" "F.Paste" "F.Mask") (roundrect_rratio 0.25) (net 1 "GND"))
  (pad "36" smd roundrect (at 4.1625 -2.75 180) (size 1.475 0.3) (layers "F.Cu" "F.Paste" "F.Mask") (roundrect_rratio 0.25) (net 4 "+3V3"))
  (pad "37" smd roundrect (at 2.75 -4.1625 180) (size 0.3 1.475) (layers "F.Cu" "F.Paste" "F.Mask") (roundrect_rratio 0.25)
   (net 30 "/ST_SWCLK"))
  (pad "38" smd roundrect (at 2.25 -4.1625 180) (size 0.3 1.475) (layers "F.Cu" "F.Paste" "F.Mask") (roundrect_rratio 0.25)
   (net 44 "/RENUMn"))
  (pad "39" smd roundrect (at 1.75 -4.1625 180) (size 0.3 1.475) (layers "F.Cu" "F.Paste" "F.Mask") (roundrect_rratio 0.25) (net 4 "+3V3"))
  (pad "40" smd roundrect (at 1.25 -4.1625 180) (size 0.3 1.475) (layers "F.Cu" "F.Paste" "F.Mask") (roundrect_rratio 0.25) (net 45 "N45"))
  (pad "41" smd roundrect (at 0.75 -4.1625 180) (size 0.3 1.475) (layers "F.Cu" "F.Paste" "F.Mask") (roundrect_rratio 0.25) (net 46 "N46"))
  (pad "42" smd roundrect (at 0.25 -4.1625 180) (size 0.3 1.475) (layers "F.Cu" "F.Paste" "F.Mask") (roundrect_rratio 0.25) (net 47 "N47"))
  (pad "43" smd roundrect (at -0.25 -4.1625 180) (size 0.3 1.475) (layers "F.Cu" "F.Paste" "F.Mask") (roundrect_rratio 0.25) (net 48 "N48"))
  (pad "44" smd roundrect (at -0.75 -4.1625 180) (size 0.3 1.475) (layers "F.Cu" "F.Paste" "F.Mask") (roundrect_rratio 0.25) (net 5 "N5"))
  (pad "45" smd roundrect (at -1.25 -4.1625 180) (size 0.3 1.475) (layers "F.Cu" "F.Paste" "F.Mask") (roundrect_rratio 0.25) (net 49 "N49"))
  (pad "46" smd roundrect (at -1.75 -4.1625 180) (size 0.3 1.475) (layers "F.Cu" "F.Paste" "F.Mask") (roundrect_rratio 0.25) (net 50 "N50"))
  (pad "47" smd roundrect (at -2.25 -4.1625 180) (size 0.3 1.475) (layers "F.Cu" "F.Paste" "F.Mask") (roundrect_rratio 0.25) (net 1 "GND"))
  (pad "48" smd roundrect (at -2.75 -4.1625 180) (size 0.3 1.475) (layers "F.Cu" "F.Paste" "F.Mask") (roundrect_rratio 0.25) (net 4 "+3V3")))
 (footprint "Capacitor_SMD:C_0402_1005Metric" (layer "F.Cu") (at 108.324994 93.849478)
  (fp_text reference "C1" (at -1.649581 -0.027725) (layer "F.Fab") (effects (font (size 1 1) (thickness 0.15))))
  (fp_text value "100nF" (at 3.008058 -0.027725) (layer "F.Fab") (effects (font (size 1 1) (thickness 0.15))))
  (fp_line (start -0.107836 0.36) (end 0.107836 0.36) (layer "F.SilkS") (width 0.12))
  (fp_line (start -0.107836 -0.36) (end 0.107836 -0.36) (layer "F.SilkS") (width 0.12))
  (pad "1" smd roundrect (at -0.48 0) (size 0.56 0.62) (layers "F.Cu" "F.Paste" "F.Mask") (roundrect_rratio 0.25) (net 3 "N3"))
  (pad "2" smd roundrect (at 0.48 0) (size 0.56 0.62) (layers "F.Cu" "F.Paste" "F.Mask") (roundrect_rratio 0.25) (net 1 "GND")))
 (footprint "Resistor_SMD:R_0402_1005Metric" (layer "F.Cu") (at 108.297605 89.933494)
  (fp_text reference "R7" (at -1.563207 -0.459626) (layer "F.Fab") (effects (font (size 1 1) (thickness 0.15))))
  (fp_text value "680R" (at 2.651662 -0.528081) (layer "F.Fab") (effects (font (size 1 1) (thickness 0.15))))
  (fp_line (start -0.153641 -0.38) (end 0.153641 -0.38) (layer "F.SilkS") (width 0.12))
  (fp_line (start -0.153641 0.38) (end 0.153641 0.38) (layer "F.SilkS") (width 0.12))
  (pad "1" smd roundrect (at -0.51 0) (size 0.54 0.64) (layers "F.Cu" "F.Paste" "F.Mask") (roundrect_rratio 0.25) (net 2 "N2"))
  (pad "2" smd roundrect (at 0.51 0) (size 0.54 0.64) (layers "F.Cu" "F.Paste" "F.Mask") (roundrect_rratio 0.25) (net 21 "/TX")))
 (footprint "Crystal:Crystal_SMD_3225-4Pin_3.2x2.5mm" (layer "B.Cu") (at 102.467158 92.072789 90)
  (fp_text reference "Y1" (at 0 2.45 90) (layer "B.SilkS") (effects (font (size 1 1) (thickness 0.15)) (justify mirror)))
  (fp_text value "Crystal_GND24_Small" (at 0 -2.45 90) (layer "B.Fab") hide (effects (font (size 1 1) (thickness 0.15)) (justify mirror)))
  (pad "1" smd rect (at -1.1 -0.85 90) (size 1.4 1.2) (layers "B.Cu" "B.Paste" "B.Mask") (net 33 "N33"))
  (pad "2" smd rect (at 1.1 -0.85 90) (size 1.4 1.2) (layers "B.Cu" "B.Paste" "B.Mask") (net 1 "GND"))
  (pad "3" smd rect (at 1.1 0.85 90) (size 1.4 1.2) (layers "B.Cu" "B.Paste" "B.Mask") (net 34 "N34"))
  (pad "4" smd rect (at -1.1 0.85 90) (size 1.4 1.2) (layers "B.Cu" "B.Paste" "B.Mask") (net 1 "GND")))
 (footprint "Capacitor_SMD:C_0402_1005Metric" (layer "B.Cu") (at 93.755858 94.912503 90)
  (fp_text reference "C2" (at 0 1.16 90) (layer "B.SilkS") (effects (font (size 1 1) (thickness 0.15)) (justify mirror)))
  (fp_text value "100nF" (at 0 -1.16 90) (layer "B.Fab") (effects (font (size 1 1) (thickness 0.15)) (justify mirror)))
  (pad "1" smd roundrect (at -0.48 0 90) (size 0.56 0.62) (layers "B.Cu" "B.Paste" "B.Mask") (roundrect_rratio 0.25) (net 11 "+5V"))
  (pad "2" smd roundrect (at 0.48 0 90) (size 0.56 0.62) (layers "B.Cu" "B.Paste" "B.Mask") (roundrect_rratio 0.25) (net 1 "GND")))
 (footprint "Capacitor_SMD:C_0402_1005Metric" (layer "B.Cu") (at 98.997563 94.889678 90)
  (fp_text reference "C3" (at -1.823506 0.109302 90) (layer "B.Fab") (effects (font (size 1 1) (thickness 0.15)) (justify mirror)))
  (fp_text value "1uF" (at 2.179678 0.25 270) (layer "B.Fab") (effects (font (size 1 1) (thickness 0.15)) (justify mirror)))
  (pad "1" smd roundrect (at -0.48 0 90) (size 0.56 0.62) (layers "B.Cu" "B.Paste" "B.Mask") (roundrect_rratio 0.25) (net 4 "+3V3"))
  (pad "2" smd roundrect (at 0.48 0 90) (size 0.56 0.62) (layers "B.Cu" "B.Paste" "B.Mask") (roundrect_rratio 0.25) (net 1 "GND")))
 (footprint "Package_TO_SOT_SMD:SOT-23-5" (layer "B.Cu") (at 96.351428 94.424751)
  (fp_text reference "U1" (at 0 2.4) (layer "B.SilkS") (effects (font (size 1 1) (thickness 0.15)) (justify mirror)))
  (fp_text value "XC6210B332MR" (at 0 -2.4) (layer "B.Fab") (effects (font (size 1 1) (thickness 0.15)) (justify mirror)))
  (pad "1" smd roundrect (at -1.1375 0.95) (size 1.325 0.6) (layers "B.Cu" "B.Paste" "B.Mask") (roundrect_rratio 0.25) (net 11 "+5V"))
  (pad "2" smd roundrect (at -1.1375 0) (size 1.325 0.6) (layers "B.Cu" "B.Paste" "B.Mask") (roundrect_rratio 0.25) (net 1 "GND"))
  (pad "3" smd roundrect (at -1.1375 -0.95) (size 1.325 0.6) (layers "B.Cu" "B.Paste" "B.Mask") (roundrect_rratio 0.25) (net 11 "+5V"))
  (pad "4" smd roundrect (at 1.1375 -0.95) (size 1.325 0.6) (layers "B.Cu" "B.Paste" "B.Mask") (roundrect_rratio 0.25) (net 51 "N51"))
  (pad "5" smd roundrect (at 1.1375 0.95) (size 1.325 0.6) (layers "B.Cu" "B.Paste" "B.Mask") (roundrect_rratio 0.25) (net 4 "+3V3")))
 (gr_rect (start 86.410911 85.09) (end 115.57 97.79) (layer "Edge.Cuts") (width 0.1) (fill none))
 (segment (start 91.360374 93.123104) (end 92.309333 94.072063) (width 0.3) (layer "F.Cu") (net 11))
 (segment (start 92.535374 94.072063) (end 93.877839 94.072063) (width 0.3) (layer "F.Cu") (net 11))
 (segment (start 95.208974 95.403198) (end 95.208974 96.122477) (width 0.3) (layer "F.Cu") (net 11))
 (segment (start 92.535374 89.272063) (end 92.009333 89.272063) (width 0.3) (layer "F.Cu") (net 11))
 (segment (start 92.309333 94.072063) (end 92.535374 94.072063) (width 0.3) (layer "F.Cu") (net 11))
 (segment (start 91.360374 89.921022) (end 91.360374 93.123104) (width 0.3) (layer "F.Cu") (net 11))
 (segment (start 92.009333 89.272063) (end 91.360374 89.921022) (width 0.3) (layer "F.Cu") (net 11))
 (segment (start 93.877839 94.072063) (end 95.208974 95.403198) (width 0.3) (layer "F.Cu") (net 11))
 (via (at 95.208974 96.122477) (size 0.8) (drill 0.4) (layers "F.Cu" "B.Cu") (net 11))
 (segment (start 95.213928 95.374751) (end 95.213928 96.117523) (width 0.3) (layer "B.Cu") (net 11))
 (segment (start 95.633535 95.374751) (end 96.226428 94.781858) (width 0.3) (layer "B.Cu") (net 11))
 (segment (start 96.226428 93.98) (end 95.721179 93.474751) (width 0.3) (layer "B.Cu") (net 11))
 (segment (start 96.226428 94.781858) (end 96.226428 93.98) (width 0.3) (layer "B.Cu") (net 11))
 (segment (start 95.213928 95.374751) (end 93.77361 95.374751) (width 0.3) (layer "B.Cu") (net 11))
 (segment (start 95.213928 96.117523) (end 95.208974 96.122477) (width 0.3) (layer "B.Cu") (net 11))
 (segment (start 95.213928 95.374751) (end 95.633535 95.374751) (width 0.3) (layer "B.Cu") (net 11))
 (segment (start 93.77361 95.374751) (end 93.755858 95.392503) (width 0.3) (layer "B.Cu") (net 11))
 (segment (start 95.721179 93.474751) (end 95.213928 93.474751) (width 0.3) (layer "B.Cu") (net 11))
 (segment (start 98.99249 95.374751) (end 98.997563 95.369678) (width 0.3) (layer "B.Cu") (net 4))
 (segment (start 97.488928 95.374751) (end 98.99249 95.374751) (width 0.3) (layer "B.Cu") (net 4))
 (segment (start 94.382202 90.610032) (end 94.382202 89.651999) (width 0.2) (layer "F.Cu") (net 17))
 (segment (start 94.382202 89.651999) (end 94.404762 89.629439) (width 0.25) (layer "F.Cu") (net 17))
 (segment (start 92.535374 91.272063) (end 92.080044 91.272063) (width 0.2) (layer "F.Cu") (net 13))
 (segment (start 92.080044 91.272063) (end 91.810374 91.541733) (width 0.2) (layer "F.Cu") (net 13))
 (segment (start 94.377166 93.565496) (end 94.377166 92.579388) (width 0.2) (layer "F.Cu") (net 13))
 (segment (start 91.810374 91.541733) (end 91.810374 92.002393) (width 0.2) (layer "F.Cu") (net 13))
 (segment (start 94.069841 92.272063) (end 94.377166 92.579388) (width 0.2) (layer "F.Cu") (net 13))
 (segment (start 91.810374 92.002393) (end 92.080044 92.272063) (width 0.2) (layer "F.Cu") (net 13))
 (segment (start 92.535374 92.272063) (end 94.069841 92.272063) (width 0.2) (layer "F.Cu") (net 13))
 (segment (start 92.080044 92.272063) (end 92.535374 92.272063) (width 0.2) (layer "F.Cu") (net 13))
 (segment (start 92.535374 90.772063) (end 92.990704 90.772063) (width 0.2) (layer "F.Cu") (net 8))
 (segment (start 92.990704 90.772063) (end 93.260374 91.041733) (width 0.2) (layer "F.Cu") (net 8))
 (segment (start 93.060374 91.772063) (end 92.535374 91.772063) (width 0.2) (layer "F.Cu") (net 8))
 (segment (start 94.374575 91.597878) (end 94.20039 91.772063) (width 0.2) (layer "F.Cu") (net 8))
 (segment (start 94.20039 91.772063) (end 92.535374 91.772063) (width 0.2) (layer "F.Cu") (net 8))
 (segment (start 93.260374 91.041733) (end 93.260374 91.572063) (width 0.2) (layer "F.Cu") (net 8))
 (segment (start 93.260374 91.572063) (end 93.060374 91.772063) (width 0.2) (layer "F.Cu") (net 8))
 (segment (start 96.4 89.42033) (end 96.4 89.209352) (width 0.2) (layer "F.Cu") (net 25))
 (segment (start 96.66967 89.69) (end 96.4 89.42033) (width 0.2) (layer "F.Cu") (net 25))
 (segment (start 95.832976 88.642328) (end 95.403624 88.642328) (width 0.2) (layer "F.Cu") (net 25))
 (segment (start 96.4 89.209352) (end 95.832976 88.642328) (width 0.2) (layer "F.Cu") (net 25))
 (segment (start 97.4375 89.69) (end 96.66967 89.69) (width 0.2) (layer "F.Cu") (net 25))
 (segment (start 96.66967 91.19) (end 96.089702 90.610032) (width 0.2) (layer "F.Cu") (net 18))
 (segment (start 96.089702 90.610032) (end 95.402202 90.610032) (width 0.2) (layer "F.Cu") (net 18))
 (segment (start 97.4375 91.19) (end 96.66967 91.19) (width 0.2) (layer "F.Cu") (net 18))
 (segment (start 97.4375 88.69) (end 96.769828 88.022328) (width 0.2) (layer "F.Cu") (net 27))
 (segment (start 95.003624 88.022328) (end 94.383624 88.642328) (width 0.2) (layer "F.Cu") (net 27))
 (segment (start 96.769828 88.022328) (end 95.003624 88.022328) (width 0.2) (layer "F.Cu") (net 27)))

